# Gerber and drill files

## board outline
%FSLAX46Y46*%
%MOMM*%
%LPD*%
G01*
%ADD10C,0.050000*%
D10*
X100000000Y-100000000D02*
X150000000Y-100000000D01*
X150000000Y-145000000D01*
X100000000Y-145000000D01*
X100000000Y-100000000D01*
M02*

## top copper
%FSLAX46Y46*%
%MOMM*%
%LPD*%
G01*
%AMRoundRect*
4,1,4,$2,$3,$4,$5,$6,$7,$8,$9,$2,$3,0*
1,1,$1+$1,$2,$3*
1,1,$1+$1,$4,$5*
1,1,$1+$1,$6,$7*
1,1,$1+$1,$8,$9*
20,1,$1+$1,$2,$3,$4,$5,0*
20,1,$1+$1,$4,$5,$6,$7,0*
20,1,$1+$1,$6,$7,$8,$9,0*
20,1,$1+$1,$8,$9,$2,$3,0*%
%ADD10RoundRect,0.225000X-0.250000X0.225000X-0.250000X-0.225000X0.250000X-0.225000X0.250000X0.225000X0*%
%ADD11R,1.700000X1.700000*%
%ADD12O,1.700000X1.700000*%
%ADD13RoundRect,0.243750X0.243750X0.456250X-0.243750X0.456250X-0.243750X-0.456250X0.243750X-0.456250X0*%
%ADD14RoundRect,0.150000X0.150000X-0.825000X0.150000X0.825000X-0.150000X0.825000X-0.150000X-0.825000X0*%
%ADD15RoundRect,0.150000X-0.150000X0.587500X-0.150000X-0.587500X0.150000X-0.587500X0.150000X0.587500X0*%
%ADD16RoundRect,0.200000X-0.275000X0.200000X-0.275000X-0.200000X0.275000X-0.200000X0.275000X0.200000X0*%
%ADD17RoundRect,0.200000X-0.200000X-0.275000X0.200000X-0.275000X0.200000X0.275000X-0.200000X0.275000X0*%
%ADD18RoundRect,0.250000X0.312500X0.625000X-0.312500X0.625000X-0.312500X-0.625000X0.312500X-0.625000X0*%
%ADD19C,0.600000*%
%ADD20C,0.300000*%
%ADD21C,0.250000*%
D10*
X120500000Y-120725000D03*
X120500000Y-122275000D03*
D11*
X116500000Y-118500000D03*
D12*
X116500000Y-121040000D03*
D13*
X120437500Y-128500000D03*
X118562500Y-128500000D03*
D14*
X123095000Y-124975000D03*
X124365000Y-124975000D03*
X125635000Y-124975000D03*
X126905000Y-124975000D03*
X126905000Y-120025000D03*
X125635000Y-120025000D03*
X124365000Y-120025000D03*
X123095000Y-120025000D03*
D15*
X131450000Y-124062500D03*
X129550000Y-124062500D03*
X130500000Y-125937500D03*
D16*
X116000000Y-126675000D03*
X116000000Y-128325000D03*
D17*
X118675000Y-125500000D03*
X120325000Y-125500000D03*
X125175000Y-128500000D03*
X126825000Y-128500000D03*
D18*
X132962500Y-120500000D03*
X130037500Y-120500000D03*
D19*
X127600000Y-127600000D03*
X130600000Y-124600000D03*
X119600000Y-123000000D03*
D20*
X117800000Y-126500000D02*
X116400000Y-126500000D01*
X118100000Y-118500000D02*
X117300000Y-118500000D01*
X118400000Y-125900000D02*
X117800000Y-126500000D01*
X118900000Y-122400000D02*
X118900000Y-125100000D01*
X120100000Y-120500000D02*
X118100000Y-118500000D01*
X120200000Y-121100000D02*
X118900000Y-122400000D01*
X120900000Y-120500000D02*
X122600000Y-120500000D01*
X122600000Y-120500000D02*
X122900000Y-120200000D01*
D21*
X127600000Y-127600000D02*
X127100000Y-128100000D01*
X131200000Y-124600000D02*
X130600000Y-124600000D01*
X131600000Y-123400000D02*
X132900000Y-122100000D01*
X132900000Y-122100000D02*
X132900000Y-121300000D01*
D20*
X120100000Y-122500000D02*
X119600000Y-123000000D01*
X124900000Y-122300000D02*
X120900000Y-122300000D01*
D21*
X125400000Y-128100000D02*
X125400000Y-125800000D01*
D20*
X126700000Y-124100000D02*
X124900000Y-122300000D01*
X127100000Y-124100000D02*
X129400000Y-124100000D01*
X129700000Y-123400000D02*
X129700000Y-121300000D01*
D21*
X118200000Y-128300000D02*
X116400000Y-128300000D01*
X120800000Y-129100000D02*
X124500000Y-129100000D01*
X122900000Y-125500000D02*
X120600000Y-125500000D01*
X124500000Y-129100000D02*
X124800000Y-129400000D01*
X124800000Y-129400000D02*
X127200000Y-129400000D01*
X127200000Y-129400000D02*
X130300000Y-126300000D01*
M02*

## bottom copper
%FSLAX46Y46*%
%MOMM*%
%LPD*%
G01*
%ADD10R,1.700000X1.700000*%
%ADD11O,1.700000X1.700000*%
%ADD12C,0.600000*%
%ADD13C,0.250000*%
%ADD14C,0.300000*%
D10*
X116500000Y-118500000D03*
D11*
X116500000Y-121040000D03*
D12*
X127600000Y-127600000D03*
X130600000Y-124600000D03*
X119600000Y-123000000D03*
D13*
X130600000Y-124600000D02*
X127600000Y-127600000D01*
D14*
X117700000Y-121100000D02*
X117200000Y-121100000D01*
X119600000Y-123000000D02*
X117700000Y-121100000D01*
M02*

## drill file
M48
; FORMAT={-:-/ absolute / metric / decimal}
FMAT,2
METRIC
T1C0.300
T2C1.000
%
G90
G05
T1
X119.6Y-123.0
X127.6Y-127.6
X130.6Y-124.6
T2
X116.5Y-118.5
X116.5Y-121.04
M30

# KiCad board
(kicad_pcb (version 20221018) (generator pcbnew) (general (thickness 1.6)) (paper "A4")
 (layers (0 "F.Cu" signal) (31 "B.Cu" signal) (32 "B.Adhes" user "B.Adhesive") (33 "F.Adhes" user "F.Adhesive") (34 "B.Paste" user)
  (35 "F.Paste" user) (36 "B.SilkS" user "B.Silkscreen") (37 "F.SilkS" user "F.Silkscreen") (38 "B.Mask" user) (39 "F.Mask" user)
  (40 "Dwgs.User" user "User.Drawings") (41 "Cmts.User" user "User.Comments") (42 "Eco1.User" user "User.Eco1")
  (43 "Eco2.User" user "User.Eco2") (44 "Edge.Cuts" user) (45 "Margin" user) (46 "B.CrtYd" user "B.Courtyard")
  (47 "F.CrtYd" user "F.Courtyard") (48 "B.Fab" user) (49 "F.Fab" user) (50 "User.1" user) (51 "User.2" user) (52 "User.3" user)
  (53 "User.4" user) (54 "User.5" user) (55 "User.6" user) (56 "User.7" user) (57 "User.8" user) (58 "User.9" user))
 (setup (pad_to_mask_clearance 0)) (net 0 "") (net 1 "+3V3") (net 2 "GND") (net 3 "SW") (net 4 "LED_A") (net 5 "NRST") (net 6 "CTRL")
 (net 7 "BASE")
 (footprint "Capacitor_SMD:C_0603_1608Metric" (layer "F.Cu") (at 120.5 121.5 -90)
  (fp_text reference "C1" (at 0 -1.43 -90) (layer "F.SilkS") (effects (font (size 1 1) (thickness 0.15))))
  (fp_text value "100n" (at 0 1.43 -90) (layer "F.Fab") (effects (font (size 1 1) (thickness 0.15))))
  (pad "1" smd roundrect (at -0.775 0 270) (size 0.9 0.95) (layers "F.Cu" "F.Paste" "F.Mask") (roundrect_rratio 0.25) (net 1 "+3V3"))
  (pad "2" smd roundrect (at 0.775 0 270) (size 0.9 0.95) (layers "F.Cu" "F.Paste" "F.Mask") (roundrect_rratio 0.25) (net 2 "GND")))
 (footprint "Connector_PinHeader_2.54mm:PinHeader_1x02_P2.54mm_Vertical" (layer "F.Cu") (at 116.5 118.5)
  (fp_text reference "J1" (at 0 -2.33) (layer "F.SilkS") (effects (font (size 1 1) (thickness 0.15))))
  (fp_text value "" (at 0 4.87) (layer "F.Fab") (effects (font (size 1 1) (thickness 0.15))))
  (pad "1" thru_hole rect (at 0 0) (size 1.7 1.7) (drill 1) (layers "*.Cu" "*.Mask") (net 1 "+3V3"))
  (pad "2" thru_hole oval (at 0 2.54) (size 1.7 1.7) (drill 1) (layers "*.Cu" "*.Mask") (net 2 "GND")))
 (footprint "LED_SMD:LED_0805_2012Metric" (layer "F.Cu") (at 119.5 128.5 180)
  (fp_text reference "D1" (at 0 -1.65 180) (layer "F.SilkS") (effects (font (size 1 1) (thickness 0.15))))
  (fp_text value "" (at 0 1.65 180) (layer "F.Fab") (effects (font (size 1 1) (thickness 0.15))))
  (pad "1" smd roundrect (at -0.9375 0 180) (size 0.975 1.4) (layers "F.Cu" "F.Paste" "F.Mask") (roundrect_rratio 0.25) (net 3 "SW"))
  (pad "2" smd roundrect (at 0.9375 0 180) (size 0.975 1.4) (layers "F.Cu" "F.Paste" "F.Mask") (roundrect_rratio 0.25) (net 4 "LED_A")))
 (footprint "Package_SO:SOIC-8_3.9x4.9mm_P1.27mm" (layer "F.Cu") (at 125 122.5 90)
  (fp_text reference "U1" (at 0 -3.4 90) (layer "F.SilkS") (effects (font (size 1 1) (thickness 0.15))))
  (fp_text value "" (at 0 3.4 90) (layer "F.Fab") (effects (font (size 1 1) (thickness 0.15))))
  (pad "1" smd roundrect (at -2.475 -1.905 90) (size 1.95 0.6) (layers "F.Cu" "F.Paste" "F.Mask") (roundrect_rratio 0.25) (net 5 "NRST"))
  (pad "2" smd roundrect (at -2.475 -0.635 90) (size 1.95 0.6) (layers "F.Cu" "F.Paste" "F.Mask") (roundrect_rratio 0.25))
  (pad "3" smd roundrect (at -2.475 0.635 90) (size 1.95 0.6) (layers "F.Cu" "F.Paste" "F.Mask") (roundrect_rratio 0.25) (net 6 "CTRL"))
  (pad "4" smd roundrect (at -2.475 1.905 90) (size 1.95 0.6) (layers "F.Cu" "F.Paste" "F.Mask") (roundrect_rratio 0.25) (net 2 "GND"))
  (pad "5" smd roundrect (at 2.475 1.905 90) (size 1.95 0.6) (layers "F.Cu" "F.Paste" "F.Mask") (roundrect_rratio 0.25))
  (pad "6" smd roundrect (at 2.475 0.635 90) (size 1.95 0.6) (layers "F.Cu" "F.Paste" "F.Mask") (roundrect_rratio 0.25))
  (pad "7" smd roundrect (at 2.475 -0.635 90) (size 1.95 0.6) (layers "F.Cu" "F.Paste" "F.Mask") (roundrect_rratio 0.25))
  (pad "8" smd roundrect (at 2.475 -1.905 90) (size 1.95 0.6) (layers "F.Cu" "F.Paste" "F.Mask") (roundrect_rratio 0.25) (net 1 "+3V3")))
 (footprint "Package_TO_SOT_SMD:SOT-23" (layer "F.Cu") (at 130.5 125 -90)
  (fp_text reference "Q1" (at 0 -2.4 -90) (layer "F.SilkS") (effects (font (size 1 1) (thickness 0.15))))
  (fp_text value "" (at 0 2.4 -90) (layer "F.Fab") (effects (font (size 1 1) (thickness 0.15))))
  (pad "1" smd roundrect (at -0.9375 -0.95 270) (size 1.475 0.6) (layers "F.Cu" "F.Paste" "F.Mask") (roundrect_rratio 0.25) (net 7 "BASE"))
  (pad "2" smd roundrect (at -0.9375 0.95 270) (size 1.475 0.6) (layers "F.Cu" "F.Paste" "F.Mask") (roundrect_rratio 0.25) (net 2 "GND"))
  (pad "3" smd roundrect (at 0.9375 0 270) (size 1.475 0.6) (layers "F.Cu" "F.Paste" "F.Mask") (roundrect_rratio 0.25) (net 3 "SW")))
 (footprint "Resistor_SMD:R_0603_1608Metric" (layer "F.Cu") (at 116 127.5 -90)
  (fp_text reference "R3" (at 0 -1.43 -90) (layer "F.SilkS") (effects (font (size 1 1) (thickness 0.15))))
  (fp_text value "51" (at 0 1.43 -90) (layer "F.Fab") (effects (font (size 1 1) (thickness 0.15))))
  (pad "1" smd roundrect (at -0.825 0 270) (size 0.8 0.95) (layers "F.Cu" "F.Paste" "F.Mask") (roundrect_rratio 0.25) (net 1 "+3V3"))
  (pad "2" smd roundrect (at 0.825 0 270) (size 0.8 0.95) (layers "F.Cu" "F.Paste" "F.Mask") (roundrect_rratio 0.25) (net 4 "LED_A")))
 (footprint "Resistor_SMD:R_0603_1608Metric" (layer "F.Cu") (at 119.5 125.5)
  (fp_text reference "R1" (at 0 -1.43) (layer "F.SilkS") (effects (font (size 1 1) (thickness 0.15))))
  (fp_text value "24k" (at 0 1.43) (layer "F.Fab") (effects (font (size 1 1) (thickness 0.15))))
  (pad "1" smd roundrect (at -0.825 0) (size 0.8 0.95) (layers "F.Cu" "F.Paste" "F.Mask") (roundrect_rratio 0.25) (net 1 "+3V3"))
  (pad "2" smd roundrect (at 0.825 0) (size 0.8 0.95) (layers "F.Cu" "F.Paste" "F.Mask") (roundrect_rratio 0.25) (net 5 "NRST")))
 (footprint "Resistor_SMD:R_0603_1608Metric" (layer "F.Cu") (at 126 128.5)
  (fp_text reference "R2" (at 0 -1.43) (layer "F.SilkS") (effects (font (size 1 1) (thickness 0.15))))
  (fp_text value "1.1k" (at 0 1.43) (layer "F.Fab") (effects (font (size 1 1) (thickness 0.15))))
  (pad "1" smd roundrect (at -0.825 0) (size 0.8 0.95) (layers "F.Cu" "F.Paste" "F.Mask") (roundrect_rratio 0.25) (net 6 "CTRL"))
  (pad "2" smd roundrect (at 0.825 0) (size 0.8 0.95) (layers "F.Cu" "F.Paste" "F.Mask") (roundrect_rratio 0.25) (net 7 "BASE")))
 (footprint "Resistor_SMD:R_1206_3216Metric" (layer "F.Cu") (at 131.5 120.5 180)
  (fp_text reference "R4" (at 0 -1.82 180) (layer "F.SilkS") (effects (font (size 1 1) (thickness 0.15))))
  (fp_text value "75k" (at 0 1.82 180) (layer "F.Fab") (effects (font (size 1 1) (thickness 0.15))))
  (pad "1" smd roundrect (at -1.4625 0 180) (size 1.125 1.75) (layers "F.Cu" "F.Paste" "F.Mask") (roundrect_rratio 0.222222) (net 7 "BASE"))
  (pad "2" smd roundrect (at 1.4625 0 180) (size 1.125 1.75) (layers "F.Cu" "F.Paste" "F.Mask") (roundrect_rratio 0.222222) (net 2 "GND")))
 (gr_rect (start 100 100) (end 150 145) (stroke (width 0.05) (type default)) (fill none) (layer "Edge.Cuts"))
 (segment (start 117.8 126.5) (end 116.4 126.5) (width 0.3) (layer "F.Cu") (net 1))
 (segment (start 118.1 118.5) (end 117.3 118.5) (width 0.3) (layer "F.Cu") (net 1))
 (segment (start 118.4 125.9) (end 117.8 126.5) (width 0.3) (layer "F.Cu") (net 1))
 (segment (start 118.9 122.4) (end 118.9 125.1) (width 0.3) (layer "F.Cu") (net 1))
 (segment (start 120.1 120.5) (end 118.1 118.5) (width 0.3) (layer "F.Cu") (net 1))
 (segment (start 120.2 121.1) (end 118.9 122.4) (width 0.3) (layer "F.Cu") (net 1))
 (segment (start 120.9 120.5) (end 122.6 120.5) (width 0.3) (layer "F.Cu") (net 1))
 (segment (start 122.6 120.5) (end 122.9 120.2) (width 0.3) (layer "F.Cu") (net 1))
 (segment (start 127.6 127.6) (end 127.1 128.1) (width 0.25) (layer "F.Cu") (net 7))
 (segment (start 131.2 124.6) (end 130.6 124.6) (width 0.25) (layer "F.Cu") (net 7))
 (segment (start 131.6 123.4) (end 132.9 122.1) (width 0.25) (layer "F.Cu") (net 7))
 (segment (start 132.9 122.1) (end 132.9 121.3) (width 0.25) (layer "F.Cu") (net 7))
 (via (at 127.6 127.6) (size 0.6) (drill 0.3) (layers "F.Cu" "B.Cu") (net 7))
 (via (at 130.6 124.6) (size 0.6) (drill 0.3) (layers "F.Cu" "B.Cu") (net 7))
 (segment (start 120.1 122.5) (end 119.6 123) (width 0.3) (layer "F.Cu") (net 2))
 (segment (start 124.9 122.3) (end 120.9 122.3) (width 0.3) (layer "F.Cu") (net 2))
 (segment (start 125.4 128.1) (end 125.4 125.8) (width 0.25) (layer "F.Cu") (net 6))
 (segment (start 126.7 124.1) (end 124.9 122.3) (width 0.3) (layer "F.Cu") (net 2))
 (segment (start 127.1 124.1) (end 129.4 124.1) (width 0.3) (layer "F.Cu") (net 2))
 (segment (start 129.7 123.4) (end 129.7 121.3) (width 0.3) (layer "F.Cu") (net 2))
 (segment (start 130.6 124.6) (end 127.6 127.6) (width 0.25) (layer "B.Cu") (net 7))
 (via (at 119.6 123) (size 0.6) (drill 0.3) (layers "F.Cu" "B.Cu") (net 2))
 (segment (start 117.7 121.1) (end 117.2 121.1) (width 0.3) (layer "B.Cu") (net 2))
 (segment (start 118.2 128.3) (end 116.4 128.3) (width 0.25) (layer "F.Cu") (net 4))
 (segment (start 119.6 123) (end 117.7 121.1) (width 0.3) (layer "B.Cu") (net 2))
 (segment (start 120.8 129.1) (end 124.5 129.1) (width 0.25) (layer "F.Cu") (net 3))
 (segment (start 122.9 125.5) (end 120.6 125.5) (width 0.25) (layer "F.Cu") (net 5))
 (segment (start 124.5 129.1) (end 124.8 129.4) (width 0.25) (layer "F.Cu") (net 3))
 (segment (start 124.8 129.4) (end 127.2 129.4) (width 0.25) (layer "F.Cu") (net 3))
 (segment (start 127.2 129.4) (end 130.3 126.3) (width 0.25) (layer "F.Cu") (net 3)))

